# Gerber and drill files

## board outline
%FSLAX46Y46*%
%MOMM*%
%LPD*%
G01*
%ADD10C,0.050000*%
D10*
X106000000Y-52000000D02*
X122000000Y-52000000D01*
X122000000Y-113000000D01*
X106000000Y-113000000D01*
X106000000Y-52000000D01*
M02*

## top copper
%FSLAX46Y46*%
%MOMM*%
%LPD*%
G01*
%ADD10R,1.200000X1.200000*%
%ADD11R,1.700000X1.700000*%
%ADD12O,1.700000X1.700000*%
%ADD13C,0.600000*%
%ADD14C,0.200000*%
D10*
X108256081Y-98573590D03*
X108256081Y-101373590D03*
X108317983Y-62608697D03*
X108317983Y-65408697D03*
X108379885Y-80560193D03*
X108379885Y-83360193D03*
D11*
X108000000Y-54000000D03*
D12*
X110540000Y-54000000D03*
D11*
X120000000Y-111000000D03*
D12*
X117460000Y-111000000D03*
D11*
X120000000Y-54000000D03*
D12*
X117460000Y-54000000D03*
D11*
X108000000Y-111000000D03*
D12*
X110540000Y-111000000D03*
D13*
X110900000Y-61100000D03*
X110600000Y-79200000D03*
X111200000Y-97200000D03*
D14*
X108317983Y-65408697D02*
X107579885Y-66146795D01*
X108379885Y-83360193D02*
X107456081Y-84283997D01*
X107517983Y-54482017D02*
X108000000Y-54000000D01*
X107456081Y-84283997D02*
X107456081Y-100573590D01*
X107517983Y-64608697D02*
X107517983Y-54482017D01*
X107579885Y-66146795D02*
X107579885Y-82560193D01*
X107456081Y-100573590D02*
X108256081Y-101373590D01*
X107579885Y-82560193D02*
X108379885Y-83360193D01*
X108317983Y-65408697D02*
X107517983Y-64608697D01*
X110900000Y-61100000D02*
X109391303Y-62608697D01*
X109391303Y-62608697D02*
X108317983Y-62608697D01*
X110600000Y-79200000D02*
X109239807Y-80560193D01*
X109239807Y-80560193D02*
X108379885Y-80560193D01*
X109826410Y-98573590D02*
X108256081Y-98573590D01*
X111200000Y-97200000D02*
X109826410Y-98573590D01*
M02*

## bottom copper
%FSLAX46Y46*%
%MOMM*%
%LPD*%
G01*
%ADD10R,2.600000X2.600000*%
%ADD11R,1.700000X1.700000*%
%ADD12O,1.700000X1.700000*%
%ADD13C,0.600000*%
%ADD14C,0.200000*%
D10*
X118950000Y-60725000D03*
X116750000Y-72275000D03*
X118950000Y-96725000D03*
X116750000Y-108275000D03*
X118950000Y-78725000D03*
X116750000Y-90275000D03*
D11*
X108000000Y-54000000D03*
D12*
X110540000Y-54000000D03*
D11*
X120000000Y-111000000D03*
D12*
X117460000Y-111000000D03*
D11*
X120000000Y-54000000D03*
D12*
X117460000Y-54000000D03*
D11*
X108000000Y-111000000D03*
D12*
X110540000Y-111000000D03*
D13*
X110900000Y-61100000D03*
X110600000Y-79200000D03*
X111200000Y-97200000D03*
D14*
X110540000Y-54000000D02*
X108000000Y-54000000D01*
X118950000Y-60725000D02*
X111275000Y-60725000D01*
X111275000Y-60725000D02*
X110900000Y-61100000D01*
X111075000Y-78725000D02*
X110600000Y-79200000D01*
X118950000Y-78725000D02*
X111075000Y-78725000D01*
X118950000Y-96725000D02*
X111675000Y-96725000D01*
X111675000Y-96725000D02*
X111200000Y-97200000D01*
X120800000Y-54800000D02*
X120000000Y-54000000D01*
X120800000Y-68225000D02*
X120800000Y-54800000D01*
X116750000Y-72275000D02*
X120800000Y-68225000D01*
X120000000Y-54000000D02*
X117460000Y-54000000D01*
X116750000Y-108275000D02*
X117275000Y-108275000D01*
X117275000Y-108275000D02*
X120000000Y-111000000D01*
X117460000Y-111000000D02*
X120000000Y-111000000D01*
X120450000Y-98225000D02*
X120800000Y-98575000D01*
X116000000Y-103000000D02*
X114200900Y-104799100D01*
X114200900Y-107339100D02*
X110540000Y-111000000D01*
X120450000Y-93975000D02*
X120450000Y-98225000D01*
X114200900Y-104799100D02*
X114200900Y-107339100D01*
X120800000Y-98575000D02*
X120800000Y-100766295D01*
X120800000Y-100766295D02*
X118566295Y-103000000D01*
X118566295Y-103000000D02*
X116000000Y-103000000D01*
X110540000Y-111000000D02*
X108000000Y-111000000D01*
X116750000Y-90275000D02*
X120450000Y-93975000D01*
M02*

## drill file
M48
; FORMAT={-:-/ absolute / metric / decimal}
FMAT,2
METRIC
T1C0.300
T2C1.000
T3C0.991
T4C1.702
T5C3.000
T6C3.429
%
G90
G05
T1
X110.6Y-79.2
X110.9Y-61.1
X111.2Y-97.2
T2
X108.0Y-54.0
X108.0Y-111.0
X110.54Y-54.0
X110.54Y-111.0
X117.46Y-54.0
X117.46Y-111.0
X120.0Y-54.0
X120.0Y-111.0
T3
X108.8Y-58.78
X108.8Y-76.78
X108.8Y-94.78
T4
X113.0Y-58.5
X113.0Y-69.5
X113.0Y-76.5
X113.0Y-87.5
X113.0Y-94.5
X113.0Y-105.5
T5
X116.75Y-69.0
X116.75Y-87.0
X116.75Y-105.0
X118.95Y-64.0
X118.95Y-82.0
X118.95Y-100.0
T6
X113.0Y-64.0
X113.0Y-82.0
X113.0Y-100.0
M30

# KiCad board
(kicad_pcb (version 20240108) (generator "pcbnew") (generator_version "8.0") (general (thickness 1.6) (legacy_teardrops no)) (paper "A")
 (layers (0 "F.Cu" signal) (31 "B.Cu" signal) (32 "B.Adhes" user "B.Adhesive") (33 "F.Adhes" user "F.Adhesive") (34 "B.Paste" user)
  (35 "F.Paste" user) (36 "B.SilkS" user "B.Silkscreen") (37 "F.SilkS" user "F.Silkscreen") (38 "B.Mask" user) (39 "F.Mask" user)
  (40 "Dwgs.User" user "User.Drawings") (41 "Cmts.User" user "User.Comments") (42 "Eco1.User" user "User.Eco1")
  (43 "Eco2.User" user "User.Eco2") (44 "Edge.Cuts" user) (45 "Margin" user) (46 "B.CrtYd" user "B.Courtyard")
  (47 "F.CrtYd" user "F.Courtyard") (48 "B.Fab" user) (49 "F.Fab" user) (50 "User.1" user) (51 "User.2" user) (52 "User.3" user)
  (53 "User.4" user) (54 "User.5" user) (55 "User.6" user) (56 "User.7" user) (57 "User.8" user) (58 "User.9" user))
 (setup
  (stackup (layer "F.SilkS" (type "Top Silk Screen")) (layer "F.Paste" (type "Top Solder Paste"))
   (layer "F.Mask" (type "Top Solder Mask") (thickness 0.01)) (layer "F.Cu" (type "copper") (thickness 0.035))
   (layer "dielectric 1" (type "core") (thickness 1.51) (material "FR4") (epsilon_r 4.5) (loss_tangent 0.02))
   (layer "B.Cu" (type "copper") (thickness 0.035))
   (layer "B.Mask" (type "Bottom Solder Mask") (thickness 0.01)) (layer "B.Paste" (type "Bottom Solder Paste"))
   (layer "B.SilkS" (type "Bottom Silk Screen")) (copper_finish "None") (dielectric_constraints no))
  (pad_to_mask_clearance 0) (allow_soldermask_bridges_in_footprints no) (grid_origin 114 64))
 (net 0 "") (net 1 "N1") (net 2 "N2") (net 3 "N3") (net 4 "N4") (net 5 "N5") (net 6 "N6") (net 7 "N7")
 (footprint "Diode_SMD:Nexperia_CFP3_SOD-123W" (layer "F.Cu") (at 108.256081 99.97359 -90)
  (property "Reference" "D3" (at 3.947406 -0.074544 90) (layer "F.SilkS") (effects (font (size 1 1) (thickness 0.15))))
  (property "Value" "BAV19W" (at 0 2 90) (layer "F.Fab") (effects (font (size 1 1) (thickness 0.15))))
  (pad "1" smd rect (at -1.4 0 270) (size 1.2 1.2) (layers "F.Cu" "F.Paste" "F.Mask") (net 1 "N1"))
  (pad "2" smd rect (at 1.4 0 270) (size 1.2 1.2) (layers "F.Cu" "F.Paste" "F.Mask") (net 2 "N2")))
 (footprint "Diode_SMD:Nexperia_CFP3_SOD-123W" (layer "F.Cu") (at 108.317983 64.008697 -90)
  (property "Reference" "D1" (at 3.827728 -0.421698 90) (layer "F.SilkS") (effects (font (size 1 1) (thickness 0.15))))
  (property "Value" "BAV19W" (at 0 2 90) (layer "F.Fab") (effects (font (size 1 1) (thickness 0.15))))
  (pad "1" smd rect (at -1.4 0 270) (size 1.2 1.2) (layers "F.Cu" "F.Paste" "F.Mask") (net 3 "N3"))
  (pad "2" smd rect (at 1.4 0 270) (size 1.2 1.2) (layers "F.Cu" "F.Paste" "F.Mask") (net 2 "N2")))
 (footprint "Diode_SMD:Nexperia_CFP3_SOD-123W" (layer "F.Cu") (at 108.379885 81.960193 -90)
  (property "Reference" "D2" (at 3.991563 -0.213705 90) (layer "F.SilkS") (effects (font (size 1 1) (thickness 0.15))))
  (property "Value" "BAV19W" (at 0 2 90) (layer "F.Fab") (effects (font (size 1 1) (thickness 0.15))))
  (pad "1" smd rect (at -1.4 0 270) (size 1.2 1.2) (layers "F.Cu" "F.Paste" "F.Mask") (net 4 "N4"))
  (pad "2" smd rect (at 1.4 0 270) (size 1.2 1.2) (layers "F.Cu" "F.Paste" "F.Mask") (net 2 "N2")))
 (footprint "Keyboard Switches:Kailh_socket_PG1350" (layer "F.Cu") (at 113 64 90)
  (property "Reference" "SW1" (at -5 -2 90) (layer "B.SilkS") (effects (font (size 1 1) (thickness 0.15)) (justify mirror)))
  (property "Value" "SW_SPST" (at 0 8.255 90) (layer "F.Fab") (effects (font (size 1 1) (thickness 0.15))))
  (pad "" np_thru_hole circle (at -5.5 0 90) (size 1.7018 1.7018) (drill 1.7018) (layers "*.Cu" "*.Mask"))
  (pad "" np_thru_hole circle (at -5 3.75 90) (size 3 3) (drill 3) (layers "*.Cu" "*.Mask"))
  (pad "" np_thru_hole circle (at 0 0 90) (size 3.429 3.429) (drill 3.429) (layers "*.Cu" "*.Mask"))
  (pad "" np_thru_hole circle (at 0 5.95 90) (size 3 3) (drill 3) (layers "*.Cu" "*.Mask"))
  (pad "" np_thru_hole circle (at 5.22 -4.2 90) (size 0.9906 0.9906) (drill 0.9906) (layers "*.Cu" "*.Mask"))
  (pad "" np_thru_hole circle (at 5.5 0 90) (size 1.7018 1.7018) (drill 1.7018) (layers "*.Cu" "*.Mask"))
  (pad "1" smd rect (at 3.275 5.95 90) (size 2.6 2.6) (layers "B.Cu" "B.Paste" "B.Mask") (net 3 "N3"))
  (pad "2" smd rect (at -8.275 3.75 90) (size 2.6 2.6) (layers "B.Cu" "B.Paste" "B.Mask") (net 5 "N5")))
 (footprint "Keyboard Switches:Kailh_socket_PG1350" (layer "F.Cu") (at 113 100 90)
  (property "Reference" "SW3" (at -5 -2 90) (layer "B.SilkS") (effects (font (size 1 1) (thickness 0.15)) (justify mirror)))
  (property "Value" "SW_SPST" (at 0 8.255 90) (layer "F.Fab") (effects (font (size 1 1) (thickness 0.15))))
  (pad "" np_thru_hole circle (at -5.5 0 90) (size 1.7018 1.7018) (drill 1.7018) (layers "*.Cu" "*.Mask"))
  (pad "" np_thru_hole circle (at -5 3.75 90) (size 3 3) (drill 3) (layers "*.Cu" "*.Mask"))
  (pad "" np_thru_hole circle (at 0 0 90) (size 3.429 3.429) (drill 3.429) (layers "*.Cu" "*.Mask"))
  (pad "" np_thru_hole circle (at 0 5.95 90) (size 3 3) (drill 3) (layers "*.Cu" "*.Mask"))
  (pad "" np_thru_hole circle (at 5.22 -4.2 90) (size 0.9906 0.9906) (drill 0.9906) (layers "*.Cu" "*.Mask"))
  (pad "" np_thru_hole circle (at 5.5 0 90) (size 1.7018 1.7018) (drill 1.7018) (layers "*.Cu" "*.Mask"))
  (pad "1" smd rect (at 3.275 5.95 90) (size 2.6 2.6) (layers "B.Cu" "B.Paste" "B.Mask") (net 1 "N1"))
  (pad "2" smd rect (at -8.275 3.75 90) (size 2.6 2.6) (layers "B.Cu" "B.Paste" "B.Mask") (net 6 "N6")))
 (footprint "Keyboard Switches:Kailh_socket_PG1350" (layer "F.Cu") (at 113 82 90)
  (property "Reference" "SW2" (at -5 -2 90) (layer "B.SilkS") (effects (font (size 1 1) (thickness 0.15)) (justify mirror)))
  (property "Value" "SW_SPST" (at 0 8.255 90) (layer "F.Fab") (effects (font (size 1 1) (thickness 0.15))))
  (pad "" np_thru_hole circle (at -5.5 0 90) (size 1.7018 1.7018) (drill 1.7018) (layers "*.Cu" "*.Mask"))
  (pad "" np_thru_hole circle (at -5 3.75 90) (size 3 3) (drill 3) (layers "*.Cu" "*.Mask"))
  (pad "" np_thru_hole circle (at 0 0 90) (size 3.429 3.429) (drill 3.429) (layers "*.Cu" "*.Mask"))
  (pad "" np_thru_hole circle (at 0 5.95 90) (size 3 3) (drill 3) (layers "*.Cu" "*.Mask"))
  (pad "" np_thru_hole circle (at 5.22 -4.2 90) (size 0.9906 0.9906) (drill 0.9906) (layers "*.Cu" "*.Mask"))
  (pad "" np_thru_hole circle (at 5.5 0 90) (size 1.7018 1.7018) (drill 1.7018) (layers "*.Cu" "*.Mask"))
  (pad "1" smd rect (at 3.275 5.95 90) (size 2.6 2.6) (layers "B.Cu" "B.Paste" "B.Mask") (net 4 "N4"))
  (pad "2" smd rect (at -8.275 3.75 90) (size 2.6 2.6) (layers "B.Cu" "B.Paste" "B.Mask") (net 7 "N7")))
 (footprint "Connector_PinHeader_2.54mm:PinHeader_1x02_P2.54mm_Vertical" (layer "B.Cu") (at 108 54 -90)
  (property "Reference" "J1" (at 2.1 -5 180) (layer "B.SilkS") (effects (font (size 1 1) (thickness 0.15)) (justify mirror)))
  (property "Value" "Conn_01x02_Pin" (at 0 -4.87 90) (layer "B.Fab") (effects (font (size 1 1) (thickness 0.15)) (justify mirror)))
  (pad "1" thru_hole rect (at 0 0 270) (size 1.7 1.7) (drill 1) (layers "*.Cu" "*.Mask") (remove_unused_layers no) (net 2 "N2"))
  (pad "2" thru_hole oval (at 0 -2.54 270) (size 1.7 1.7) (drill 1) (layers "*.Cu" "*.Mask") (remove_unused_layers no) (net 2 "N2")))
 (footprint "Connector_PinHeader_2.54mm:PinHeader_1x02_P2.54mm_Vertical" (layer "B.Cu") (at 120 111 90)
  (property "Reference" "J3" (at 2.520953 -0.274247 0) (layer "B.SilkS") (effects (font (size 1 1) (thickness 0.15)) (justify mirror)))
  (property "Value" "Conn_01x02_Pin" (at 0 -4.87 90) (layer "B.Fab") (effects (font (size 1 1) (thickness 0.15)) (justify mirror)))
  (pad "1" thru_hole rect (at 0 0 90) (size 1.7 1.7) (drill 1) (layers "*.Cu" "*.Mask") (remove_unused_layers no) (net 6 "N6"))
  (pad "2" thru_hole oval (at 0 -2.54 90) (size 1.7 1.7) (drill 1) (layers "*.Cu" "*.Mask") (remove_unused_layers no) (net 6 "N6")))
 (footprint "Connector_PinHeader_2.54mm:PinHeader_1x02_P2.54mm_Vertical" (layer "B.Cu") (at 120 54 90)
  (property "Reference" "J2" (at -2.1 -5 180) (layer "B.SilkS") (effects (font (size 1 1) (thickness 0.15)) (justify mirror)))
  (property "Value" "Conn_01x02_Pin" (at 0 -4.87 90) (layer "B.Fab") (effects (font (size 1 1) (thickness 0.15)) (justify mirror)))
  (pad "1" thru_hole rect (at 0 0 90) (size 1.7 1.7) (drill 1) (layers "*.Cu" "*.Mask") (remove_unused_layers no) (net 5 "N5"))
  (pad "2" thru_hole oval (at 0 -2.54 90) (size 1.7 1.7) (drill 1) (layers "*.Cu" "*.Mask") (remove_unused_layers no) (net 5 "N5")))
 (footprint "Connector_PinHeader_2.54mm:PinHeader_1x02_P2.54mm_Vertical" (layer "B.Cu") (at 108 111 -90)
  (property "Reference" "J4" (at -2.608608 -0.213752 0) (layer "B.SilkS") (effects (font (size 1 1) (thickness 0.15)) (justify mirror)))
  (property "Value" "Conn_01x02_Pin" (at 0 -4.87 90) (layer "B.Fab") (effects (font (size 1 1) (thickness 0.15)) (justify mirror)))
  (pad "1" thru_hole rect (at 0 0 270) (size 1.7 1.7) (drill 1) (layers "*.Cu" "*.Mask") (remove_unused_layers no) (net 7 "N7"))
  (pad "2" thru_hole oval (at 0 -2.54 270) (size 1.7 1.7) (drill 1) (layers "*.Cu" "*.Mask") (remove_unused_layers no) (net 7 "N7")))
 (gr_rect (start 106 52) (end 122 113) (stroke (width 0.05) (type default)) (fill none) (layer "Edge.Cuts"))
 (segment (start 108.317983 65.408697) (end 107.579885 66.146795) (width 0.2) (layer "F.Cu") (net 2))
 (segment (start 108.379885 83.360193) (end 107.456081 84.283997) (width 0.2) (layer "F.Cu") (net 2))
 (segment (start 107.517983 54.482017) (end 108 54) (width 0.2) (layer "F.Cu") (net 2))
 (segment (start 107.456081 84.283997) (end 107.456081 100.57359) (width 0.2) (layer "F.Cu") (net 2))
 (segment (start 107.517983 64.608697) (end 107.517983 54.482017) (width 0.2) (layer "F.Cu") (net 2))
 (segment (start 107.579885 66.146795) (end 107.579885 82.560193) (width 0.2) (layer "F.Cu") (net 2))
 (segment (start 107.456081 100.57359) (end 108.256081 101.37359) (width 0.2) (layer "F.Cu") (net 2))
 (segment (start 107.579885 82.560193) (end 108.379885 83.360193) (width 0.2) (layer "F.Cu") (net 2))
 (segment (start 108.317983 65.408697) (end 107.517983 64.608697) (width 0.2) (layer "F.Cu") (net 2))
 (segment (start 110.54 54) (end 108 54) (width 0.2) (layer "B.Cu") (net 2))
 (segment (start 110.9 61.1) (end 109.391303 62.608697) (width 0.2) (layer "F.Cu") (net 3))
 (segment (start 109.391303 62.608697) (end 108.317983 62.608697) (width 0.2) (layer "F.Cu") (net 3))
 (via (at 110.9 61.1) (size 0.6) (drill 0.3) (layers "F.Cu" "B.Cu") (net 3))
 (segment (start 118.95 60.725) (end 111.275 60.725) (width 0.2) (layer "B.Cu") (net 3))
 (segment (start 111.275 60.725) (end 110.9 61.1) (width 0.2) (layer "B.Cu") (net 3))
 (segment (start 110.6 79.2) (end 109.239807 80.560193) (width 0.2) (layer "F.Cu") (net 4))
 (segment (start 109.239807 80.560193) (end 108.379885 80.560193) (width 0.2) (layer "F.Cu") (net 4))
 (via (at 110.6 79.2) (size 0.6) (drill 0.3) (layers "F.Cu" "B.Cu") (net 4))
 (segment (start 111.075 78.725) (end 110.6 79.2) (width 0.2) (layer "B.Cu") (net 4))
 (segment (start 118.95 78.725) (end 111.075 78.725) (width 0.2) (layer "B.Cu") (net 4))
 (segment (start 109.82641 98.57359) (end 108.256081 98.57359) (width 0.2) (layer "F.Cu") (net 1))
 (segment (start 111.2 97.2) (end 109.82641 98.57359) (width 0.2) (layer "F.Cu") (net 1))
 (via (at 111.2 97.2) (size 0.6) (drill 0.3) (layers "F.Cu" "B.Cu") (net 1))
 (segment (start 118.95 96.725) (end 111.675 96.725) (width 0.2) (layer "B.Cu") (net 1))
 (segment (start 111.675 96.725) (end 111.2 97.2) (width 0.2) (layer "B.Cu") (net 1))
 (segment (start 120.8 54.8) (end 120 54) (width 0.2) (layer "B.Cu") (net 5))
 (segment (start 120.8 68.225) (end 120.8 54.8) (width 0.2) (layer "B.Cu") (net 5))
 (segment (start 116.75 72.275) (end 120.8 68.225) (width 0.2) (layer "B.Cu") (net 5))
 (segment (start 120 54) (end 117.46 54) (width 0.2) (layer "B.Cu") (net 5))
 (segment (start 116.75 108.275) (end 117.275 108.275) (width 0.2) (layer "B.Cu") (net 6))
 (segment (start 117.275 108.275) (end 120 111) (width 0.2) (layer "B.Cu") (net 6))
 (segment (start 117.46 111) (end 120 111) (width 0.2) (layer "B.Cu") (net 6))
 (segment (start 120.45 98.225) (end 120.8 98.575) (width 0.2) (layer "B.Cu") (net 7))
 (segment (start 116 103) (end 114.2009 104.7991) (width 0.2) (layer "B.Cu") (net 7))
 (segment (start 114.2009 107.3391) (end 110.54 111) (width 0.2) (layer "B.Cu") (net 7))
 (segment (start 120.45 93.975) (end 120.45 98.225) (width 0.2) (layer "B.Cu") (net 7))
 (segment (start 114.2009 104.7991) (end 114.2009 107.3391) (width 0.2) (layer "B.Cu") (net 7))
 (segment (start 120.8 98.575) (end 120.8 100.766295) (width 0.2) (layer "B.Cu") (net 7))
 (segment (start 120.8 100.766295) (end 118.566295 103) (width 0.2) (layer "B.Cu") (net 7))
 (segment (start 118.566295 103) (end 116 103) (width 0.2) (layer "B.Cu") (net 7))
 (segment (start 110.54 111) (end 108 111) (width 0.2) (layer "B.Cu") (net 7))
 (segment (start 116.75 90.275) (end 120.45 93.975) (width 0.2) (layer "B.Cu") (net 7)))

